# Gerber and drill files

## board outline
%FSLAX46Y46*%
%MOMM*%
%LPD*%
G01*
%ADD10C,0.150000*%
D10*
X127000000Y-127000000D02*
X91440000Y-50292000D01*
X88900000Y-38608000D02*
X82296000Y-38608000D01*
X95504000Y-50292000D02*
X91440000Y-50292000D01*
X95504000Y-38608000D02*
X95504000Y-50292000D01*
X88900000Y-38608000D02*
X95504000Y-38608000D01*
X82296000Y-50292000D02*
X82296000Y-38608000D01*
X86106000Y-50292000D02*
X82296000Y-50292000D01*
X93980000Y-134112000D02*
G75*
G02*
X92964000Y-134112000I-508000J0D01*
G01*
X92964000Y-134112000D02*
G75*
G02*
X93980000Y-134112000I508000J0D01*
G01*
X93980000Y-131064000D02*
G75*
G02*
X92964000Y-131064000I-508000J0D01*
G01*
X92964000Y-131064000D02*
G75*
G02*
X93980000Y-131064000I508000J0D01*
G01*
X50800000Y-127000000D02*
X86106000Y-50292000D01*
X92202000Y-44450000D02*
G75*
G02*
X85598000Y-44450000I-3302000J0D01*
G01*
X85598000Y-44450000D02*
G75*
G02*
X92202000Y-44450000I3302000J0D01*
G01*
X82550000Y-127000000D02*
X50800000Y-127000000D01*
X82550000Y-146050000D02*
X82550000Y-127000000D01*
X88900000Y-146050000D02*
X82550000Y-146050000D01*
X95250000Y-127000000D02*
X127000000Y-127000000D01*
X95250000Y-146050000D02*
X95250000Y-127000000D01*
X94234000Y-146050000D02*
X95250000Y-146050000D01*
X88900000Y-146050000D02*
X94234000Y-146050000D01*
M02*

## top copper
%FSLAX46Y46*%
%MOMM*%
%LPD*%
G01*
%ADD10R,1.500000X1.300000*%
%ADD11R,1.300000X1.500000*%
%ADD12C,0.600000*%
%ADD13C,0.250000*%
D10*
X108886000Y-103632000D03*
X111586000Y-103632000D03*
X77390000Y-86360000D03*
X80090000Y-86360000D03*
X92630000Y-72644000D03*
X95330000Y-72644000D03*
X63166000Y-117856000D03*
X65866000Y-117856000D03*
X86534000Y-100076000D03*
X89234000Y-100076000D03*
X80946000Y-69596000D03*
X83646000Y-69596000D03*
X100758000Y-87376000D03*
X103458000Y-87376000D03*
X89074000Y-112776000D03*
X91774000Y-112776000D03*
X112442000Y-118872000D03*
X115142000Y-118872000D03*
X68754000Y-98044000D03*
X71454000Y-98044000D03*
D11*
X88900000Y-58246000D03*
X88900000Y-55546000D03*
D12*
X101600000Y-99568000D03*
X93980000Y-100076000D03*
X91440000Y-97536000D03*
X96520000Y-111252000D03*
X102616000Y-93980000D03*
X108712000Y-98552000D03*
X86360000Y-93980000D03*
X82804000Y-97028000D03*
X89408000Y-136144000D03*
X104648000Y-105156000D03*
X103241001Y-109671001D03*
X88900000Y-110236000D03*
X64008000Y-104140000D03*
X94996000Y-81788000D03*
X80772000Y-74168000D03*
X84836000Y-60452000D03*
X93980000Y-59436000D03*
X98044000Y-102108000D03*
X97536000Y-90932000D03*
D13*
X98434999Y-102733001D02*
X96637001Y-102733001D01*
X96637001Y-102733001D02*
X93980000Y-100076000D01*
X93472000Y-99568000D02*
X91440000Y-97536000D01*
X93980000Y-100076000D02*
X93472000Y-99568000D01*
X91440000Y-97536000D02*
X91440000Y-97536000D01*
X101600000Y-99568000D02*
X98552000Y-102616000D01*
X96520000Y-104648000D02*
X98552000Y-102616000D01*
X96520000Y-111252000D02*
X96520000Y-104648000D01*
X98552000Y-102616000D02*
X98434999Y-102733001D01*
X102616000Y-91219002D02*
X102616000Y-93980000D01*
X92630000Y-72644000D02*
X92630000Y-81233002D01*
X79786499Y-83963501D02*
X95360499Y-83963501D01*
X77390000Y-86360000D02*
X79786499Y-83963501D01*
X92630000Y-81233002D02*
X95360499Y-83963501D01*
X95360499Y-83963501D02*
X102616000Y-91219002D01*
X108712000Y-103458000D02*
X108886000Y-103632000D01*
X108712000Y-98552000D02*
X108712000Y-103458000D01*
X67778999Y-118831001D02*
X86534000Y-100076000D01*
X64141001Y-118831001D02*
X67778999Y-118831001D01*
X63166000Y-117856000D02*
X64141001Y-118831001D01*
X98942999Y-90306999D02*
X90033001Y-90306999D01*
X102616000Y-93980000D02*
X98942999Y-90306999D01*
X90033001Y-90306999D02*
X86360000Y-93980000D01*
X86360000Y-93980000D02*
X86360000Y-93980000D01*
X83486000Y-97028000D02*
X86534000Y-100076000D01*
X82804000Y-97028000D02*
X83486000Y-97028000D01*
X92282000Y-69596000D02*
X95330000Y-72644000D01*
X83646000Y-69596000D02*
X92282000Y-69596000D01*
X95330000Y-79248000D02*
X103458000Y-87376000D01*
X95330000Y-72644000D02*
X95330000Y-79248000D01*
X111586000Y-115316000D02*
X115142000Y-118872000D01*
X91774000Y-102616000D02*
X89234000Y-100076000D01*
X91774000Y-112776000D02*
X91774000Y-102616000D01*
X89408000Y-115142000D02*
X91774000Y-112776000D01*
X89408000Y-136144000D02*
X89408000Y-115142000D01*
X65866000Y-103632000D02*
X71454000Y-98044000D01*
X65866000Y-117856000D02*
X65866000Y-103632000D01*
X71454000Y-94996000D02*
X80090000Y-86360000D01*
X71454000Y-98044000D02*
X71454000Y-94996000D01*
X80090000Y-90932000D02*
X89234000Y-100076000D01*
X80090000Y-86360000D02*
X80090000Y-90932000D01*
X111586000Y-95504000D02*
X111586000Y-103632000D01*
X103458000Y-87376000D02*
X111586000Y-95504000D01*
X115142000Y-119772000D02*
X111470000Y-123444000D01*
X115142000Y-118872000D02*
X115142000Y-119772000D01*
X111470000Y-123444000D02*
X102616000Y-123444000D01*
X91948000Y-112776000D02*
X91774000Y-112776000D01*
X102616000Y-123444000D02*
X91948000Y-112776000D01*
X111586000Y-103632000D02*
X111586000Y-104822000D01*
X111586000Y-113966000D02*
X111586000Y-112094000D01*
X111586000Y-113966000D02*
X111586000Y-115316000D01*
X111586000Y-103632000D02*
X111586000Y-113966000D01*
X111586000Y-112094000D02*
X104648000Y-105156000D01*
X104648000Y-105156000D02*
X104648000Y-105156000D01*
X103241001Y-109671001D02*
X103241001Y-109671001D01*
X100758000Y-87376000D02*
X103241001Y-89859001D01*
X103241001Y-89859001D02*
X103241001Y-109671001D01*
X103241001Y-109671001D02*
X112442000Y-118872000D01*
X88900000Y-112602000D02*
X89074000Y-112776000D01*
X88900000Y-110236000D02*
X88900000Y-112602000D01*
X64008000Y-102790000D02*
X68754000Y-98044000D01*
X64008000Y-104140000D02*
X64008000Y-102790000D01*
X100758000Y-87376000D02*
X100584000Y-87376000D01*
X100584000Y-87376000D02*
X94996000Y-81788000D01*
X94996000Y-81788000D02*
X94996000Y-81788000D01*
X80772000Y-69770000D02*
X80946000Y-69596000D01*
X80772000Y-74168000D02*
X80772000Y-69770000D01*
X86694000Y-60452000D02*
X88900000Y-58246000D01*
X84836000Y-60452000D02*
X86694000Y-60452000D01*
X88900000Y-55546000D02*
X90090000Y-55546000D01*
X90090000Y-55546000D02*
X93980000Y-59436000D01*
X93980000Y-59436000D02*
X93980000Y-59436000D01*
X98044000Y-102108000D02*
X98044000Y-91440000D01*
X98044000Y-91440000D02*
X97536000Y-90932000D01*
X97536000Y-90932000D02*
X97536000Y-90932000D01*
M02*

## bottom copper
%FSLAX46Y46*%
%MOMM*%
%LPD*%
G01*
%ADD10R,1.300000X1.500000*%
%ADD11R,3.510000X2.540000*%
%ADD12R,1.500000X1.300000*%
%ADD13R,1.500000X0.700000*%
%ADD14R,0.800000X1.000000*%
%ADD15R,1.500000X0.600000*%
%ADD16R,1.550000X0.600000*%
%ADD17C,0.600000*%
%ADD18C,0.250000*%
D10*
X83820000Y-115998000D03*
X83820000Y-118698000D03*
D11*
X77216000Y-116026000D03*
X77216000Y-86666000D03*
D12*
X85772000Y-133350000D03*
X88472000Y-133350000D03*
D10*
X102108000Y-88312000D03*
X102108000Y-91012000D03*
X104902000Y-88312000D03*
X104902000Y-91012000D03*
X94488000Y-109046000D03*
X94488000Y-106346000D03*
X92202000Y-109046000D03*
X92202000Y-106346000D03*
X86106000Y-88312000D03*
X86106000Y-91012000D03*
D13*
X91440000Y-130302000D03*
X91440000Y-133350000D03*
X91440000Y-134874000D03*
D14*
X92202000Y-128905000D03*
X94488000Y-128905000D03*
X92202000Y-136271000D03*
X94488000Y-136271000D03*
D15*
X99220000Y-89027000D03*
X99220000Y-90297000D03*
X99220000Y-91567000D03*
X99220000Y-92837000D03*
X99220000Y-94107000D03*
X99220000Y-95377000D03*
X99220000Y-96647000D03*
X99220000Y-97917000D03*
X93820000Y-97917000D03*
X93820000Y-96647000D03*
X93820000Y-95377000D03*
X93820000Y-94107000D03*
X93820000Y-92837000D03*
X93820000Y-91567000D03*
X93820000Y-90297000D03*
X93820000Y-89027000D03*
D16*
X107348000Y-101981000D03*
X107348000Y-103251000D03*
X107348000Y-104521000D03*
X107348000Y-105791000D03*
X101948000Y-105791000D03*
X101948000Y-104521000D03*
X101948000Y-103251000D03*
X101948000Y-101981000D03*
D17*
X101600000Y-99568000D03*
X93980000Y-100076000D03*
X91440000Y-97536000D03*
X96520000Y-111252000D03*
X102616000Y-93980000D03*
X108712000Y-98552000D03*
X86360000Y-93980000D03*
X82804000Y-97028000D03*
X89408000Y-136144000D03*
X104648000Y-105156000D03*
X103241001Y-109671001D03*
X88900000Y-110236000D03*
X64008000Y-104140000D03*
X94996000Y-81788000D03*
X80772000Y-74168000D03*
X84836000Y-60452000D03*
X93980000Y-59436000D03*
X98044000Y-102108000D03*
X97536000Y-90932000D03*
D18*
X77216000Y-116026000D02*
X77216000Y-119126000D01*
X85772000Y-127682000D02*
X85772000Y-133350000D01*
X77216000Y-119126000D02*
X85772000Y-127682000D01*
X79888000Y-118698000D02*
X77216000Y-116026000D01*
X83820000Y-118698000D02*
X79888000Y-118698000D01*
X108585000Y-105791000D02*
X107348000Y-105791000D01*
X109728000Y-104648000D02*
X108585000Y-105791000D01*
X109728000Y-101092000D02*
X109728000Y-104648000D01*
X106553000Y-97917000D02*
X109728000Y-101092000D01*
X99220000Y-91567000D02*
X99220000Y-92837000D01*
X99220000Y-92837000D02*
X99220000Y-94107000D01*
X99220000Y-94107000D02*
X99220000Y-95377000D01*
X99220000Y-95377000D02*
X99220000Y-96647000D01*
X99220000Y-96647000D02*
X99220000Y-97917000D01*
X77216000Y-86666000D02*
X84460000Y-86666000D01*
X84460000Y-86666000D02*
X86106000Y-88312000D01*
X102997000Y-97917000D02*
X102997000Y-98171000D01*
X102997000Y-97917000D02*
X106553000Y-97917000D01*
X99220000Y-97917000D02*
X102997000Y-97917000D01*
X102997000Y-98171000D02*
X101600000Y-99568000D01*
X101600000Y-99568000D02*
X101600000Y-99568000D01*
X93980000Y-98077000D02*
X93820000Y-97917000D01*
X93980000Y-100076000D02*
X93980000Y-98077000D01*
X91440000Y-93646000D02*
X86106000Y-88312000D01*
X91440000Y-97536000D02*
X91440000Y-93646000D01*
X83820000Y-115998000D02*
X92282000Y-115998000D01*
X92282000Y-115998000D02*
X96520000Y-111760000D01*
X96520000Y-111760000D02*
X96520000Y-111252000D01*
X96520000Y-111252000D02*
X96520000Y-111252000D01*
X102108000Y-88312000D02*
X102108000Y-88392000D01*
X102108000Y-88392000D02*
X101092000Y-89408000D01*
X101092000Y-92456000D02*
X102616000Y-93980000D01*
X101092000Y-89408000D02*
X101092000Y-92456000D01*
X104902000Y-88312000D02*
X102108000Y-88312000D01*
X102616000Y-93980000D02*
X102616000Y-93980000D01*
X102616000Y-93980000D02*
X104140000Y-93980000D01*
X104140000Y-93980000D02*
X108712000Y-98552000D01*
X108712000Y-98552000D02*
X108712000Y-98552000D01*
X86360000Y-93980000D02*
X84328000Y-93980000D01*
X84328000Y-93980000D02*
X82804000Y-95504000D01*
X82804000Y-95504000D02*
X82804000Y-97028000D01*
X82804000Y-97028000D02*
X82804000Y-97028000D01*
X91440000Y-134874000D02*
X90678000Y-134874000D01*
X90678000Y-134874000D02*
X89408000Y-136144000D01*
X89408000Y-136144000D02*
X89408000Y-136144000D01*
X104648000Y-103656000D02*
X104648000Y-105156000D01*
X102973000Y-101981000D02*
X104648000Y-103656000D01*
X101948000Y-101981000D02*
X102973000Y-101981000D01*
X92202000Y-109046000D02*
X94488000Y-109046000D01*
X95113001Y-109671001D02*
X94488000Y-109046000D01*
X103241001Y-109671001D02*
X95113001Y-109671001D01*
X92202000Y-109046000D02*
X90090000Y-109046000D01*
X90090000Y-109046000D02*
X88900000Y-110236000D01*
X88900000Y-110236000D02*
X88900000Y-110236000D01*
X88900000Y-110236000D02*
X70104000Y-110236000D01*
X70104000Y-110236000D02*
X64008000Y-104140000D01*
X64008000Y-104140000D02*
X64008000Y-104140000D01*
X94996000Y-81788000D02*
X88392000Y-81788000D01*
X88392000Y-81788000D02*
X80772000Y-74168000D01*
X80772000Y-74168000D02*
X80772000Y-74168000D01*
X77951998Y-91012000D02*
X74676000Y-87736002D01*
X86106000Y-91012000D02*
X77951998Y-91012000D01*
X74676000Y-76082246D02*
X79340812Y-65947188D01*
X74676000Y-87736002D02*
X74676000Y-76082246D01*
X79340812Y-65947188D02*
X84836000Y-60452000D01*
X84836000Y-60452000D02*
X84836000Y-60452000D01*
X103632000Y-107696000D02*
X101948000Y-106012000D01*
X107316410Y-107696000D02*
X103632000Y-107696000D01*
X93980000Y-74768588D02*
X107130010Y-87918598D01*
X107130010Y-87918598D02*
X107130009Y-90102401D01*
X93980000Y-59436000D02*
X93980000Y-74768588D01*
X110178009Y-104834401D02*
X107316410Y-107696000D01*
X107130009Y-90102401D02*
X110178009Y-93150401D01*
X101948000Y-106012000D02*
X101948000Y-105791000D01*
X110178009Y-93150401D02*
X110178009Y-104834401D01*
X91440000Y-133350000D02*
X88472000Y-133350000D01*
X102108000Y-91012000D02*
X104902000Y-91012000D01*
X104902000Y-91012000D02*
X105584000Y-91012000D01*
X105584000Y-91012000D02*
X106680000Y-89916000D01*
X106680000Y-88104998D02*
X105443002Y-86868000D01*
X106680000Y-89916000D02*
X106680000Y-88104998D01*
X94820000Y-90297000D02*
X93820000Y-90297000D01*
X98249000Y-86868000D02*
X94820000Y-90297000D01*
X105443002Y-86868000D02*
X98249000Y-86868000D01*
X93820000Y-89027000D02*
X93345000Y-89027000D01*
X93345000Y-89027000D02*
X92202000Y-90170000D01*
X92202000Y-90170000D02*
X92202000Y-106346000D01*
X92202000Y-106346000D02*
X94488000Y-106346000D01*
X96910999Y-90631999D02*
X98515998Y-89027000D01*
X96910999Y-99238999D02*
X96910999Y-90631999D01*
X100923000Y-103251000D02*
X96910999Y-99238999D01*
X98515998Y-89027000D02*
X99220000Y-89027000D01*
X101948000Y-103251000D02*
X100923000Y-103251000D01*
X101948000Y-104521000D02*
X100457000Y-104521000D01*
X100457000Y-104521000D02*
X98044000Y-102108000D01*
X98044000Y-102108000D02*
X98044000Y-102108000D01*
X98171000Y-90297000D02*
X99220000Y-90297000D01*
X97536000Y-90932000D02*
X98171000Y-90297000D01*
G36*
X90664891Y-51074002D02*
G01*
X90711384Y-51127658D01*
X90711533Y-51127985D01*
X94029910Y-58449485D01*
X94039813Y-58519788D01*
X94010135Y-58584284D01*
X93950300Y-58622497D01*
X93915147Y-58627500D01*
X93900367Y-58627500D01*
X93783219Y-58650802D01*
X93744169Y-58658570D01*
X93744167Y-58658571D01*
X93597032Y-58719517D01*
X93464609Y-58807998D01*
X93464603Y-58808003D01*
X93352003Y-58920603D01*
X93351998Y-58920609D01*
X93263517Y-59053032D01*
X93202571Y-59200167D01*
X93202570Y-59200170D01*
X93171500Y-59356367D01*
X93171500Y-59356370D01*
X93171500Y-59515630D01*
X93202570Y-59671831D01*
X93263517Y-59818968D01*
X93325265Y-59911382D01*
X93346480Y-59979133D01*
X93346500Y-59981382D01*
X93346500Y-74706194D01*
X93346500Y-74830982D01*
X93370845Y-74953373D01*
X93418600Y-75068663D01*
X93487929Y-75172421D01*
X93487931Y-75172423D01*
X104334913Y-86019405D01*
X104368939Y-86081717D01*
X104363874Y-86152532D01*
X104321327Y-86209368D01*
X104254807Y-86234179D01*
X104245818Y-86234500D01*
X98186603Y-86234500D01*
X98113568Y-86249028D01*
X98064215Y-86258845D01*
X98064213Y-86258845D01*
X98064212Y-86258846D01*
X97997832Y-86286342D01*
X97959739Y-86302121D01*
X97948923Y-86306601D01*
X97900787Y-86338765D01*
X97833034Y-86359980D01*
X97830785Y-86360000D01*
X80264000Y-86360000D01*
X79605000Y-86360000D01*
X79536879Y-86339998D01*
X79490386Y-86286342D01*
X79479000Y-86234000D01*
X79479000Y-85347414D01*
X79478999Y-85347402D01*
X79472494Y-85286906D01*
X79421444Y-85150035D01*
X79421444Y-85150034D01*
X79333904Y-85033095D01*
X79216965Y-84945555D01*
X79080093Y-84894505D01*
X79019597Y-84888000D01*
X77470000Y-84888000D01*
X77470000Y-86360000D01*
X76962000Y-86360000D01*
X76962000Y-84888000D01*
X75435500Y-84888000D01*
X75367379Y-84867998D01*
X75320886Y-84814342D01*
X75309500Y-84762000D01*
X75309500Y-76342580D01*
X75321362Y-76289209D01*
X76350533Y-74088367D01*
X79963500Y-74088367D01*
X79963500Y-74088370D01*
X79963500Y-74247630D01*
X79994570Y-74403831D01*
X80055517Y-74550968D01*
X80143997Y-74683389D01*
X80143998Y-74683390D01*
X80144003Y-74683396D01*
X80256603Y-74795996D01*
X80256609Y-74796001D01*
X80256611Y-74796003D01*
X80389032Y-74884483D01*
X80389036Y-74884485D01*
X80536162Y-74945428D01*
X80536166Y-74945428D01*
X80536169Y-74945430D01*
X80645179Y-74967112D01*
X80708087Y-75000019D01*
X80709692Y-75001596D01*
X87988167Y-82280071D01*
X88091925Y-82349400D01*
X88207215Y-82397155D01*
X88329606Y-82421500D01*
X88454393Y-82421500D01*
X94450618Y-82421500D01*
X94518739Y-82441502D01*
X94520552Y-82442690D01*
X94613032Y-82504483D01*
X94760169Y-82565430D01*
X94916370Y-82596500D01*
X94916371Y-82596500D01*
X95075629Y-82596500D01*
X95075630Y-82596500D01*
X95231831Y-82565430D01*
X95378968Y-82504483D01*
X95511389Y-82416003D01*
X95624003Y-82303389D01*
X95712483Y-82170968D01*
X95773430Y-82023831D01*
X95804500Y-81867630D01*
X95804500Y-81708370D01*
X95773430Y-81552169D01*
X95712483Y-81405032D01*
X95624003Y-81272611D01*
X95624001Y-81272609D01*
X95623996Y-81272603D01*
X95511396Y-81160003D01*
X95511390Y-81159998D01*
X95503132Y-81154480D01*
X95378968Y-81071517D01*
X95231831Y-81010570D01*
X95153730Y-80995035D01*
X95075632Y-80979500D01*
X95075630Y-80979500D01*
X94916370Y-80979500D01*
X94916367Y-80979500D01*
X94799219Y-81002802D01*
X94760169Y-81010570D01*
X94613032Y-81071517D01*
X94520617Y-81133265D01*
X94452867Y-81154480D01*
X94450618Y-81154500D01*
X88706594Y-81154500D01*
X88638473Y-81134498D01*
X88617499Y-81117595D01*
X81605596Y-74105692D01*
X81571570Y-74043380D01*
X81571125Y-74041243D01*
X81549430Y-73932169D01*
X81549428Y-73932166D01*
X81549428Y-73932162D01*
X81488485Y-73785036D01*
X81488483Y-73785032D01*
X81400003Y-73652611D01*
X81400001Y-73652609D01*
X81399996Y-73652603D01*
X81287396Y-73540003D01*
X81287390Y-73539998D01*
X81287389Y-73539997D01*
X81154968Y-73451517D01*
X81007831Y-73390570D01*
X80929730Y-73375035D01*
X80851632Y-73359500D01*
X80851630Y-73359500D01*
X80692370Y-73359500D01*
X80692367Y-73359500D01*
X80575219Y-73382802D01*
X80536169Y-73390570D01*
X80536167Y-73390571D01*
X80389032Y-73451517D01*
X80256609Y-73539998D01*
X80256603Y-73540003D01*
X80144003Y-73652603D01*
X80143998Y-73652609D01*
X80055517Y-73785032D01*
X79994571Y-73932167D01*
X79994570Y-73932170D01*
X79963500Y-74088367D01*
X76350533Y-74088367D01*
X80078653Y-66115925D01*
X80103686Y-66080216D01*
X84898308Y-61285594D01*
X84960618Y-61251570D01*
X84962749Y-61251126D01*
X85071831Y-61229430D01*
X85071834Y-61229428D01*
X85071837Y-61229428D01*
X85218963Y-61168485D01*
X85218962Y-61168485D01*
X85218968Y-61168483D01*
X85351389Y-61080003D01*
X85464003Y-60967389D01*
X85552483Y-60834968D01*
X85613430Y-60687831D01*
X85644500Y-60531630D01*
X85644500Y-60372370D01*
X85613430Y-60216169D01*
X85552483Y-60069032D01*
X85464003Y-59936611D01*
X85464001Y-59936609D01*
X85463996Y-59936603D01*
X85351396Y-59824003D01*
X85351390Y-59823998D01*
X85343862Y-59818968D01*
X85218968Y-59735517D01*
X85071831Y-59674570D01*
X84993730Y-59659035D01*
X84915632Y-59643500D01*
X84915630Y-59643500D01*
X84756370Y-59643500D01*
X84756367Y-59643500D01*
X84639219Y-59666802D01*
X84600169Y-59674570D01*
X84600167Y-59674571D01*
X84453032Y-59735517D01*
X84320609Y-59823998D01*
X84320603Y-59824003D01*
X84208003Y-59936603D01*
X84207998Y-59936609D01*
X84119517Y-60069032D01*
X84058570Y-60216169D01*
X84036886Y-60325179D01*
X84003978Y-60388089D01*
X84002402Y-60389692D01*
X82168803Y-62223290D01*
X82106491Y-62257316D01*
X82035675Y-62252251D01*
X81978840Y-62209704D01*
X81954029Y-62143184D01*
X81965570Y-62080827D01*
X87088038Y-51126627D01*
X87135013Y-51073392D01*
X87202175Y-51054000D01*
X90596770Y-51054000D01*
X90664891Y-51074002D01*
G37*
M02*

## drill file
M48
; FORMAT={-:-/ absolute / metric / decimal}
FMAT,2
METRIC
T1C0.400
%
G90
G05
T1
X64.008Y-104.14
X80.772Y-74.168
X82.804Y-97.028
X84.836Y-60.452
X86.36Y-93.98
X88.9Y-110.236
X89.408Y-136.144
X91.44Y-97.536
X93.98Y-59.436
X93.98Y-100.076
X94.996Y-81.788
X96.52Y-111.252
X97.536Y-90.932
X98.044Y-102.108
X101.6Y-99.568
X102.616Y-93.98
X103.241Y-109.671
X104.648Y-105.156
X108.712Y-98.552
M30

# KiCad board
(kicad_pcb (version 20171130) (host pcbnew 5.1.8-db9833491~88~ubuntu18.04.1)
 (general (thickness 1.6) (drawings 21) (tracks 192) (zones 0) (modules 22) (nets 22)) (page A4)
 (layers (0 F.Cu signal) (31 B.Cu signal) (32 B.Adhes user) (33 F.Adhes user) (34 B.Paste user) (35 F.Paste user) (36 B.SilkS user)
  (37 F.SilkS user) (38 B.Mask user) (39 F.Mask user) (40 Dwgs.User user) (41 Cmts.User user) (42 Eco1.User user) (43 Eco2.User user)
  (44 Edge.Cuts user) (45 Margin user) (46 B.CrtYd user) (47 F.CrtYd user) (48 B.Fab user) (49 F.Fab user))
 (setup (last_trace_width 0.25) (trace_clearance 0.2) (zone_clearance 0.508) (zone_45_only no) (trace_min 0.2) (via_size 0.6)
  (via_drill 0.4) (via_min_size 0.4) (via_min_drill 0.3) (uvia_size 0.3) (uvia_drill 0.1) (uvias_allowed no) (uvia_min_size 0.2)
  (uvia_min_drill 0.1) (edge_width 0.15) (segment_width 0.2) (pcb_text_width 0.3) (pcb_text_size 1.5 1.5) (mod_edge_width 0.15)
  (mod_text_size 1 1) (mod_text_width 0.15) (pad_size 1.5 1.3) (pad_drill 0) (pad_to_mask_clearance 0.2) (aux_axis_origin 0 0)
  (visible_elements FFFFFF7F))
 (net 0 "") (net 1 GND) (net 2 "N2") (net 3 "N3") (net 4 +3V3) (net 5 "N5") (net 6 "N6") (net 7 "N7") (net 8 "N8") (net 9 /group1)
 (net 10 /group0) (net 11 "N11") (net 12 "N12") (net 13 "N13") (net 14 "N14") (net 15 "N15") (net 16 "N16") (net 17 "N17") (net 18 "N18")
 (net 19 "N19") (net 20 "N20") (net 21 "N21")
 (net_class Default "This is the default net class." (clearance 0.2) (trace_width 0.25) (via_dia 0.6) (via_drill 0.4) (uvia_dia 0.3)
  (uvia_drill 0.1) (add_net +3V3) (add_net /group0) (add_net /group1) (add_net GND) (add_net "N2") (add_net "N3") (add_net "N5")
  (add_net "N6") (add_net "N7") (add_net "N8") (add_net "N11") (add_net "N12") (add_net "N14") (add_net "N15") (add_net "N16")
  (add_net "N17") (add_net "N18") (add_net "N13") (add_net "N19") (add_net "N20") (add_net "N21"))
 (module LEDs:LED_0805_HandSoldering (layer B.Cu) (at 83.82 117.348 90)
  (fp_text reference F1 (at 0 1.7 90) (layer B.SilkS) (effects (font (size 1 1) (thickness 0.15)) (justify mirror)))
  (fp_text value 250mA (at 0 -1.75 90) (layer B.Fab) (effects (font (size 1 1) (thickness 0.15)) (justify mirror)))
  (pad 2 smd rect (at 1.35 0 90) (size 1.5 1.3) (layers B.Cu B.Paste B.Mask) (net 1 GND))
  (pad 1 smd rect (at -1.35 0 90) (size 1.5 1.3) (layers B.Cu B.Paste B.Mask) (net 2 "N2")))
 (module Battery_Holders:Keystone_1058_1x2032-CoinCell (layer B.Cu) (at 77.216 101.346 90)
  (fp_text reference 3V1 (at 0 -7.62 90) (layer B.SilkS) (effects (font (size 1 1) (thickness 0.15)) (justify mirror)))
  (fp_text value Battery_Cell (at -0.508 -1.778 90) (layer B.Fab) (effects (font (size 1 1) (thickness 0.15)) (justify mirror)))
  (pad 1 smd rect (at -14.68 0 90) (size 2.54 3.51) (layers B.Cu B.Paste B.Mask) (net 2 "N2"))
  (pad 2 smd rect (at 14.68 0 90) (size 2.54 3.51) (layers B.Cu B.Paste B.Mask) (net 1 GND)))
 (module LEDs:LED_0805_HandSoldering (layer F.Cu) (at 110.236 103.632)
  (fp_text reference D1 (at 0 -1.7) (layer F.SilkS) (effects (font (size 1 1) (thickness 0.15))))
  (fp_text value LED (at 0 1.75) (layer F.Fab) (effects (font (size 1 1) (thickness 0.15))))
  (pad 1 smd rect (at -1.35 0) (size 1.5 1.3) (layers F.Cu F.Paste F.Mask) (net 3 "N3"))
  (pad 2 smd rect (at 1.35 0) (size 1.5 1.3) (layers F.Cu F.Paste F.Mask) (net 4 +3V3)))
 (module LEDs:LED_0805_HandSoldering (layer F.Cu) (at 78.74 86.36)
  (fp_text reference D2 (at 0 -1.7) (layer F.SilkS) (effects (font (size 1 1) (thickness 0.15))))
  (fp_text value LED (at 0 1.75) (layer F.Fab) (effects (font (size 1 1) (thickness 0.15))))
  (pad 1 smd rect (at -1.35 0) (size 1.5 1.3) (layers F.Cu F.Paste F.Mask) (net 3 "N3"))
  (pad 2 smd rect (at 1.35 0) (size 1.5 1.3) (layers F.Cu F.Paste F.Mask) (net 4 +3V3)))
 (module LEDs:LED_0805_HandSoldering (layer F.Cu) (at 93.98 72.644)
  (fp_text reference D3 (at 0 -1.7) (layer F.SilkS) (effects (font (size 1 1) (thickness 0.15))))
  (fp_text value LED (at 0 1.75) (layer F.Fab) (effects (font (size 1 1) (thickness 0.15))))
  (pad 1 smd rect (at -1.35 0) (size 1.5 1.3) (layers F.Cu F.Paste F.Mask) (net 3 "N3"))
  (pad 2 smd rect (at 1.35 0) (size 1.5 1.3) (layers F.Cu F.Paste F.Mask) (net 4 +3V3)))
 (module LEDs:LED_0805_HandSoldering (layer F.Cu) (at 64.516 117.856)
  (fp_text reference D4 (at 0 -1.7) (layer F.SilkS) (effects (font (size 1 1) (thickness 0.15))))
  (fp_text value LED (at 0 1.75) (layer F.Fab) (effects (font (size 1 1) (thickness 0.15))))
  (pad 1 smd rect (at -1.35 0) (size 1.5 1.3) (layers F.Cu F.Paste F.Mask) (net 3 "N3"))
  (pad 2 smd rect (at 1.35 0) (size 1.5 1.3) (layers F.Cu F.Paste F.Mask) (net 4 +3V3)))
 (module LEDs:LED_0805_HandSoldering (layer F.Cu) (at 87.884 100.076)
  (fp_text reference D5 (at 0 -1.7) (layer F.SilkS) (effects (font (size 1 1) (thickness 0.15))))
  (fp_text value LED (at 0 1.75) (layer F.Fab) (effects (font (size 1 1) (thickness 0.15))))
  (pad 1 smd rect (at -1.35 0) (size 1.5 1.3) (layers F.Cu F.Paste F.Mask) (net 3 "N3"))
  (pad 2 smd rect (at 1.35 0) (size 1.5 1.3) (layers F.Cu F.Paste F.Mask) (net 4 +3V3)))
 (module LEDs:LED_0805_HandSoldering (layer F.Cu) (at 82.296 69.596)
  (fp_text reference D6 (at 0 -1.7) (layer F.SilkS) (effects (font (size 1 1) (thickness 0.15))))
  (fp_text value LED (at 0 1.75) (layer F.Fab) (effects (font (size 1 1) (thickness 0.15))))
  (pad 1 smd rect (at -1.35 0) (size 1.5 1.3) (layers F.Cu F.Paste F.Mask) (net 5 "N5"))
  (pad 2 smd rect (at 1.35 0) (size 1.5 1.3) (layers F.Cu F.Paste F.Mask) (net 4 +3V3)))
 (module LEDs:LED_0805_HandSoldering (layer F.Cu) (at 102.108 87.376)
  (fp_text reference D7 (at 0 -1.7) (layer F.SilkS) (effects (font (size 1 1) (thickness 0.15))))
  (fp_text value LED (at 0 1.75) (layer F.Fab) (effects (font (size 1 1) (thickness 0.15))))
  (pad 1 smd rect (at -1.35 0) (size 1.5 1.3) (layers F.Cu F.Paste F.Mask) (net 5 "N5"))
  (pad 2 smd rect (at 1.35 0) (size 1.5 1.3) (layers F.Cu F.Paste F.Mask) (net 4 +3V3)))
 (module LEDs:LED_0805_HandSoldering (layer F.Cu) (at 90.424 112.776)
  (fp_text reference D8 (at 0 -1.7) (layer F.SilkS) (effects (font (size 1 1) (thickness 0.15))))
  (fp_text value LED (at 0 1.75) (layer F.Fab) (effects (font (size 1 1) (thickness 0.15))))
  (pad 1 smd rect (at -1.35 0) (size 1.5 1.3) (layers F.Cu F.Paste F.Mask) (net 5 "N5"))
  (pad 2 smd rect (at 1.35 0) (size 1.5 1.3) (layers F.Cu F.Paste F.Mask) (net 4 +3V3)))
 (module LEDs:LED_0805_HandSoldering (layer F.Cu) (at 113.792 118.872)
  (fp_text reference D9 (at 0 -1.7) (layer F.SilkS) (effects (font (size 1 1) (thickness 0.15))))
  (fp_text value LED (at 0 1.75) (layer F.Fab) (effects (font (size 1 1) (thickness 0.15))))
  (pad 1 smd rect (at -1.35 0) (size 1.5 1.3) (layers F.Cu F.Paste F.Mask) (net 5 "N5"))
  (pad 2 smd rect (at 1.35 0) (size 1.5 1.3) (layers F.Cu F.Paste F.Mask) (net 4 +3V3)))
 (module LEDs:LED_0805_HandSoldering (layer F.Cu) (at 70.104 98.044)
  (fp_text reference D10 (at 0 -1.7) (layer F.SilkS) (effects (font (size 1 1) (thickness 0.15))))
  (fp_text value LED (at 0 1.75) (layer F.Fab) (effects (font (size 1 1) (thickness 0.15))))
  (pad 1 smd rect (at -1.35 0) (size 1.5 1.3) (layers F.Cu F.Paste F.Mask) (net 5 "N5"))
  (pad 2 smd rect (at 1.35 0) (size 1.5 1.3) (layers F.Cu F.Paste F.Mask) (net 4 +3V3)))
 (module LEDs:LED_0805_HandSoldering (layer F.Cu) (at 88.9 56.896 90)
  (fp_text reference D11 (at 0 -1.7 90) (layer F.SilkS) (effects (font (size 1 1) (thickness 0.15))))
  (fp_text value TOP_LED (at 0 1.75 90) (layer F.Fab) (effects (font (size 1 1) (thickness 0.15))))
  (pad 1 smd rect (at -1.35 0 90) (size 1.5 1.3) (layers F.Cu F.Paste F.Mask) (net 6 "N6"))
  (pad 2 smd rect (at 1.35 0 90) (size 1.5 1.3) (layers F.Cu F.Paste F.Mask) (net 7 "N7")))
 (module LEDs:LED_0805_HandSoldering (layer B.Cu) (at 87.122 133.35)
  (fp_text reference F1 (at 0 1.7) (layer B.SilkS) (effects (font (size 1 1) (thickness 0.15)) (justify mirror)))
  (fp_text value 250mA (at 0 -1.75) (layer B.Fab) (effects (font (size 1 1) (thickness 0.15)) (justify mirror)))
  (pad 1 smd rect (at -1.35 0) (size 1.5 1.3) (layers B.Cu B.Paste B.Mask) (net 2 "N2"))
  (pad 2 smd rect (at 1.35 0) (size 1.5 1.3) (layers B.Cu B.Paste B.Mask) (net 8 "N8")))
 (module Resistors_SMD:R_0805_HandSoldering (layer B.Cu) (at 102.108 89.662 270)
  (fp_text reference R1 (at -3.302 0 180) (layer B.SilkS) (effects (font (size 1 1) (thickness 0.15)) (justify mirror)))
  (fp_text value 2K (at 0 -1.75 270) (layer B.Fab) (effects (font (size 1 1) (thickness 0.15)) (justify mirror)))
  (pad 1 smd rect (at -1.35 0 270) (size 1.5 1.3) (layers B.Cu B.Paste B.Mask) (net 3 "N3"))
  (pad 2 smd rect (at 1.35 0 270) (size 1.5 1.3) (layers B.Cu B.Paste B.Mask) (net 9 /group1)))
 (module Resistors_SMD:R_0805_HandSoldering (layer B.Cu) (at 104.902 89.662 270)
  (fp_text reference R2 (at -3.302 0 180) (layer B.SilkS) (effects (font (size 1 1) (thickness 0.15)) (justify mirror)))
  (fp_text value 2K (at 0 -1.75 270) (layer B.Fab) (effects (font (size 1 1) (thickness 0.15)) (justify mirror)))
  (pad 1 smd rect (at -1.35 0 270) (size 1.5 1.3) (layers B.Cu B.Paste B.Mask) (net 3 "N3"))
  (pad 2 smd rect (at 1.35 0 270) (size 1.5 1.3) (layers B.Cu B.Paste B.Mask) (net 9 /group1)))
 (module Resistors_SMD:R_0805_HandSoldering (layer B.Cu) (at 94.488 107.696 90)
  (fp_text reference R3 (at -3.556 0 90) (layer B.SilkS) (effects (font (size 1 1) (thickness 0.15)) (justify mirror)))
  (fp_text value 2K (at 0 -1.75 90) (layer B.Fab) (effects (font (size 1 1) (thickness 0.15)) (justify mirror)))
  (pad 1 smd rect (at -1.35 0 90) (size 1.5 1.3) (layers B.Cu B.Paste B.Mask) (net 5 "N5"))
  (pad 2 smd rect (at 1.35 0 90) (size 1.5 1.3) (layers B.Cu B.Paste B.Mask) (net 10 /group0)))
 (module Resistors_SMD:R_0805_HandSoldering (layer B.Cu) (at 92.202 107.696 90)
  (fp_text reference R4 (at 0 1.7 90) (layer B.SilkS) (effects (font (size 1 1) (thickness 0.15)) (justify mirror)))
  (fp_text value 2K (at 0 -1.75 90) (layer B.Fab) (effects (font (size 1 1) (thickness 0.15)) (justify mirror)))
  (pad 1 smd rect (at -1.35 0 90) (size 1.5 1.3) (layers B.Cu B.Paste B.Mask) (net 5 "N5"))
  (pad 2 smd rect (at 1.35 0 90) (size 1.5 1.3) (layers B.Cu B.Paste B.Mask) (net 10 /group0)))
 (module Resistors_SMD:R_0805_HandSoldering (layer B.Cu) (at 86.106 89.662 270)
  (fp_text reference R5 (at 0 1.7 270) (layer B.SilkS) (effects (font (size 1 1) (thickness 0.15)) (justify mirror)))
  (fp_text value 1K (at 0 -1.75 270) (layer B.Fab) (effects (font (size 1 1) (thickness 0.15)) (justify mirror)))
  (pad 1 smd rect (at -1.35 0 270) (size 1.5 1.3) (layers B.Cu B.Paste B.Mask) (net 1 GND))
  (pad 2 smd rect (at 1.35 0 270) (size 1.5 1.3) (layers B.Cu B.Paste B.Mask) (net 6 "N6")))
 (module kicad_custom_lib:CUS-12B (layer B.Cu) (at 96.266 132.588 270)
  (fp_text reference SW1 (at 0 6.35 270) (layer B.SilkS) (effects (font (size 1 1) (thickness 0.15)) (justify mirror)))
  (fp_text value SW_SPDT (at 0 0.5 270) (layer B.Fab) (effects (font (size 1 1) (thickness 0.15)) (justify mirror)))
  (pad 1 smd rect (at -2.286 4.826 270) (size 0.7 1.5) (layers B.Cu B.Paste B.Mask) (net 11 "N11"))
  (pad 2 smd rect (at 0.762 4.826 270) (size 0.7 1.5) (layers B.Cu B.Paste B.Mask) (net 8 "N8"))
  (pad 3 smd rect (at 2.286 4.826 270) (size 0.7 1.5) (layers B.Cu B.Paste B.Mask) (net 4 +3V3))
  (pad 4 smd rect (at -3.683 4.064 270) (size 1 0.8) (layers B.Cu B.Paste B.Mask))
  (pad 5 smd rect (at -3.683 1.778 270) (size 1 0.8) (layers B.Cu B.Paste B.Mask))
  (pad 6 smd rect (at 3.683 4.064 270) (size 1 0.8) (layers B.Cu B.Paste B.Mask))
  (pad 7 smd rect (at 3.683 1.778 270) (size 1 0.8) (layers B.Cu B.Paste B.Mask)))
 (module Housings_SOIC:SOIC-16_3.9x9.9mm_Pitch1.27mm (layer B.Cu) (at 96.52 93.472 180)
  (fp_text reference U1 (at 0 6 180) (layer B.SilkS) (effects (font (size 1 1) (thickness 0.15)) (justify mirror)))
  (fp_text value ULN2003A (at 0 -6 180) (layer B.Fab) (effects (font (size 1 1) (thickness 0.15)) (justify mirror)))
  (pad 1 smd rect (at -2.7 4.445 180) (size 1.5 0.6) (layers B.Cu B.Paste B.Mask) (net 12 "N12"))
  (pad 2 smd rect (at -2.7 3.175 180) (size 1.5 0.6) (layers B.Cu B.Paste B.Mask) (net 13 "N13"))
  (pad 3 smd rect (at -2.7 1.905 180) (size 1.5 0.6) (layers B.Cu B.Paste B.Mask) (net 1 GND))
  (pad 4 smd rect (at -2.7 0.635 180) (size 1.5 0.6) (layers B.Cu B.Paste B.Mask) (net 1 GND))
  (pad 5 smd rect (at -2.7 -0.635 180) (size 1.5 0.6) (layers B.Cu B.Paste B.Mask) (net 1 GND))
  (pad 6 smd rect (at -2.7 -1.905 180) (size 1.5 0.6) (layers B.Cu B.Paste B.Mask) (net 1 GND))
  (pad 7 smd rect (at -2.7 -3.175 180) (size 1.5 0.6) (layers B.Cu B.Paste B.Mask) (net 1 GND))
  (pad 8 smd rect (at -2.7 -4.445 180) (size 1.5 0.6) (layers B.Cu B.Paste B.Mask) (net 1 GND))
  (pad 9 smd rect (at 2.7 -4.445 180) (size 1.5 0.6) (layers B.Cu B.Paste B.Mask) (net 1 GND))
  (pad 10 smd rect (at 2.7 -3.175 180) (size 1.5 0.6) (layers B.Cu B.Paste B.Mask) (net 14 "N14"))
  (pad 11 smd rect (at 2.7 -1.905 180) (size 1.5 0.6) (layers B.Cu B.Paste B.Mask) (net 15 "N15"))
  (pad 12 smd rect (at 2.7 -0.635 180) (size 1.5 0.6) (layers B.Cu B.Paste B.Mask) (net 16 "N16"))
  (pad 13 smd rect (at 2.7 0.635 180) (size 1.5 0.6) (layers B.Cu B.Paste B.Mask) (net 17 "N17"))
  (pad 14 smd rect (at 2.7 1.905 180) (size 1.5 0.6) (layers B.Cu B.Paste B.Mask) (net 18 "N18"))
  (pad 15 smd rect (at 2.7 3.175 180) (size 1.5 0.6) (layers B.Cu B.Paste B.Mask) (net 9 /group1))
  (pad 16 smd rect (at 2.7 4.445 180) (size 1.5 0.6) (layers B.Cu B.Paste B.Mask) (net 10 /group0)))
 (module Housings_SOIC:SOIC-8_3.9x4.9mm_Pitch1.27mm (layer B.Cu) (at 104.648 103.886 180)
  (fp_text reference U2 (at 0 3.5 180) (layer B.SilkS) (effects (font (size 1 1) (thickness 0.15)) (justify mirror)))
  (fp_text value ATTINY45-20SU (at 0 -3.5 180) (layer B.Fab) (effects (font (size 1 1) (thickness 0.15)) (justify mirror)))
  (pad 1 smd rect (at -2.7 1.905 180) (size 1.55 0.6) (layers B.Cu B.Paste B.Mask) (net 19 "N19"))
  (pad 2 smd rect (at -2.7 0.635 180) (size 1.55 0.6) (layers B.Cu B.Paste B.Mask) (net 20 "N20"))
  (pad 3 smd rect (at -2.7 -0.635 180) (size 1.55 0.6) (layers B.Cu B.Paste B.Mask) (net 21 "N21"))
  (pad 4 smd rect (at -2.7 -1.905 180) (size 1.55 0.6) (layers B.Cu B.Paste B.Mask) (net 1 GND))
  (pad 5 smd rect (at 2.7 -1.905 180) (size 1.55 0.6) (layers B.Cu B.Paste B.Mask) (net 7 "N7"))
  (pad 6 smd rect (at 2.7 -0.635 180) (size 1.55 0.6) (layers B.Cu B.Paste B.Mask) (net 13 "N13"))
  (pad 7 smd rect (at 2.7 0.635 180) (size 1.55 0.6) (layers B.Cu B.Paste B.Mask) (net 12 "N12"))
  (pad 8 smd rect (at 2.7 1.905 180) (size 1.55 0.6) (layers B.Cu B.Paste B.Mask) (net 4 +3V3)))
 (gr_line (start 127 127) (end 91.44 50.292) (layer Edge.Cuts) (width 0.15))
 (gr_line (start 88.9 38.608) (end 82.296 38.608) (layer Edge.Cuts) (width 0.15))
 (gr_line (start 95.504 50.292) (end 91.44 50.292) (layer Edge.Cuts) (width 0.15))
 (gr_line (start 95.504 38.608) (end 95.504 50.292) (layer Edge.Cuts) (width 0.15))
 (gr_line (start 88.9 38.608) (end 95.504 38.608) (layer Edge.Cuts) (width 0.15))
 (gr_line (start 82.296 50.292) (end 82.296 38.608) (layer Edge.Cuts) (width 0.15))
 (gr_line (start 86.106 50.292) (end 82.296 50.292) (layer Edge.Cuts) (width 0.15))
 (gr_circle (center 93.472 134.112) (end 93.472 133.604) (layer Edge.Cuts) (width 0.15))
 (gr_circle (center 93.472 131.064) (end 92.964 131.064) (layer Edge.Cuts) (width 0.15))
 (gr_line (start 50.8 127) (end 86.106 50.292) (angle 90) (layer Edge.Cuts) (width 0.15))
 (gr_circle (center 88.9 44.45) (end 88.9 41.148) (layer Edge.Cuts) (width 0.15))
 (gr_line (start 82.55 127) (end 50.8 127) (angle 90) (layer Edge.Cuts) (width 0.15))
 (gr_line (start 82.55 146.05) (end 82.55 127) (angle 90) (layer Edge.Cuts) (width 0.15))
 (gr_line (start 88.9 146.05) (end 82.55 146.05) (angle 90) (layer Edge.Cuts) (width 0.15))
 (gr_line (start 95.25 127) (end 127 127) (angle 90) (layer Edge.Cuts) (width 0.15))
 (gr_line (start 95.25 146.05) (end 95.25 127) (angle 90) (layer Edge.Cuts) (width 0.15))
 (gr_line (start 94.234 146.05) (end 95.25 146.05) (angle 90) (layer Edge.Cuts) (width 0.15))
 (gr_line (start 88.9 146.05) (end 94.234 146.05) (angle 90) (layer Edge.Cuts) (width 0.15))
 (segment (start 77.216 116.026) (end 77.216 119.126) (width 0.25) (layer B.Cu) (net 2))
 (segment (start 85.772 127.682) (end 85.772 133.35) (width 0.25) (layer B.Cu) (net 2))
 (segment (start 77.216 119.126) (end 85.772 127.682) (width 0.25) (layer B.Cu) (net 2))
 (segment (start 79.888 118.698) (end 77.216 116.026) (width 0.25) (layer B.Cu) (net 2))
 (segment (start 83.82 118.698) (end 79.888 118.698) (width 0.25) (layer B.Cu) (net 2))
 (segment (start 108.585 105.791) (end 107.348 105.791) (width 0.25) (layer B.Cu) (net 1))
 (segment (start 109.728 104.648) (end 108.585 105.791) (width 0.25) (layer B.Cu) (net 1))
 (segment (start 109.728 101.092) (end 109.728 104.648) (width 0.25) (layer B.Cu) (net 1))
 (segment (start 106.553 97.917) (end 109.728 101.092) (width 0.25) (layer B.Cu) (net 1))
 (segment (start 99.22 91.567) (end 99.22 92.837) (width 0.25) (layer B.Cu) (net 1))
 (segment (start 99.22 92.837) (end 99.22 94.107) (width 0.25) (layer B.Cu) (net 1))
 (segment (start 99.22 94.107) (end 99.22 95.377) (width 0.25) (layer B.Cu) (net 1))
 (segment (start 99.22 95.377) (end 99.22 96.647) (width 0.25) (layer B.Cu) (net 1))
 (segment (start 99.22 96.647) (end 99.22 97.917) (width 0.25) (layer B.Cu) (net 1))
 (segment (start 77.216 86.666) (end 84.46 86.666) (width 0.25) (layer B.Cu) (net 1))
 (segment (start 84.46 86.666) (end 86.106 88.312) (width 0.25) (layer B.Cu) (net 1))
 (segment (start 102.997 97.917) (end 102.997 98.171) (width 0.25) (layer B.Cu) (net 1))
 (segment (start 102.997 97.917) (end 106.553 97.917) (width 0.25) (layer B.Cu) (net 1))
 (segment (start 99.22 97.917) (end 102.997 97.917) (width 0.25) (layer B.Cu) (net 1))
 (segment (start 102.997 98.171) (end 101.6 99.568) (width 0.25) (layer B.Cu) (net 1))
 (segment (start 101.6 99.568) (end 101.6 99.568) (width 0.25) (layer B.Cu) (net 1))
 (via (at 101.6 99.568) (size 0.6) (drill 0.4) (layers F.Cu B.Cu) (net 1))
 (segment (start 98.434999 102.733001) (end 96.637001 102.733001) (width 0.25) (layer F.Cu) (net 1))
 (segment (start 96.637001 102.733001) (end 93.98 100.076) (width 0.25) (layer F.Cu) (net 1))
 (segment (start 93.472 99.568) (end 91.44 97.536) (width 0.25) (layer F.Cu) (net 1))
 (segment (start 93.98 100.076) (end 93.472 99.568) (width 0.25) (layer F.Cu) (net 1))
 (via (at 93.98 100.076) (size 0.6) (drill 0.4) (layers F.Cu B.Cu) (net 1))
 (segment (start 91.44 97.536) (end 91.44 97.536) (width 0.25) (layer F.Cu) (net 1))
 (via (at 91.44 97.536) (size 0.6) (drill 0.4) (layers F.Cu B.Cu) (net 1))
 (segment (start 93.98 98.077) (end 93.82 97.917) (width 0.25) (layer B.Cu) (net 1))
 (segment (start 93.98 100.076) (end 93.98 98.077) (width 0.25) (layer B.Cu) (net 1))
 (segment (start 91.44 93.646) (end 86.106 88.312) (width 0.25) (layer B.Cu) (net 1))
 (segment (start 91.44 97.536) (end 91.44 93.646) (width 0.25) (layer B.Cu) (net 1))
 (segment (start 83.82 115.998) (end 92.282 115.998) (width 0.25) (layer B.Cu) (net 1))
 (segment (start 92.282 115.998) (end 96.52 111.76) (width 0.25) (layer B.Cu) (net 1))
 (segment (start 96.52 111.76) (end 96.52 111.252) (width 0.25) (layer B.Cu) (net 1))
 (segment (start 96.52 111.252) (end 96.52 111.252) (width 0.25) (layer B.Cu) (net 1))
 (via (at 96.52 111.252) (size 0.6) (drill 0.4) (layers F.Cu B.Cu) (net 1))
 (segment (start 101.6 99.568) (end 98.552 102.616) (width 0.25) (layer F.Cu) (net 1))
 (segment (start 96.52 104.648) (end 98.552 102.616) (width 0.25) (layer F.Cu) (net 1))
 (segment (start 96.52 111.252) (end 96.52 104.648) (width 0.25) (layer F.Cu) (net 1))
 (segment (start 98.552 102.616) (end 98.434999 102.733001) (width 0.25) (layer F.Cu) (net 1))
 (segment (start 102.108 88.312) (end 102.108 88.392) (width 0.25) (layer B.Cu) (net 3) (status C00000))
 (segment (start 102.108 88.392) (end 101.092 89.408) (width 0.25) (layer B.Cu) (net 3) (status 400000))
 (segment (start 101.092 92.456) (end 102.616 93.98) (width 0.25) (layer B.Cu) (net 3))
 (segment (start 101.092 89.408) (end 101.092 92.456) (width 0.25) (layer B.Cu) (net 3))
 (segment (start 104.902 88.312) (end 102.108 88.312) (width 0.25) (layer B.Cu) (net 3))
 (segment (start 102.616 93.98) (end 102.616 93.98) (width 0.25) (layer B.Cu) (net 3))
 (via (at 102.616 93.98) (size 0.6) (drill 0.4) (layers F.Cu B.Cu) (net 3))
 (segment (start 102.616 91.219002) (end 102.616 93.98) (width 0.25) (layer F.Cu) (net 3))
 (segment (start 92.63 72.644) (end 92.63 81.233002) (width 0.25) (layer F.Cu) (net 3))
 (segment (start 79.786499 83.963501) (end 95.360499 83.963501) (width 0.25) (layer F.Cu) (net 3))
 (segment (start 77.39 86.36) (end 79.786499 83.963501) (width 0.25) (layer F.Cu) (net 3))
 (segment (start 92.63 81.233002) (end 95.360499 83.963501) (width 0.25) (layer F.Cu) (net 3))
 (segment (start 95.360499 83.963501) (end 102.616 91.219002) (width 0.25) (layer F.Cu) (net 3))
 (segment (start 102.616 93.98) (end 104.14 93.98) (width 0.25) (layer B.Cu) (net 3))
 (segment (start 104.14 93.98) (end 108.712 98.552) (width 0.25) (layer B.Cu) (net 3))
 (segment (start 108.712 98.552) (end 108.712 98.552) (width 0.25) (layer B.Cu) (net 3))
 (via (at 108.712 98.552) (size 0.6) (drill 0.4) (layers F.Cu B.Cu) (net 3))
 (segment (start 108.712 103.458) (end 108.886 103.632) (width 0.25) (layer F.Cu) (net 3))
 (segment (start 108.712 98.552) (end 108.712 103.458) (width 0.25) (layer F.Cu) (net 3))
 (segment (start 67.778999 118.831001) (end 86.534 100.076) (width 0.25) (layer F.Cu) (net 3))
 (segment (start 64.141001 118.831001) (end 67.778999 118.831001) (width 0.25) (layer F.Cu) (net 3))
 (segment (start 63.166 117.856) (end 64.141001 118.831001) (width 0.25) (layer F.Cu) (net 3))
 (segment (start 98.942999 90.306999) (end 90.033001 90.306999) (width 0.25) (layer F.Cu) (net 3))
 (segment (start 102.616 93.98) (end 98.942999 90.306999) (width 0.25) (layer F.Cu) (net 3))
 (segment (start 90.033001 90.306999) (end 86.36 93.98) (width 0.25) (layer F.Cu) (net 3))
 (segment (start 86.36 93.98) (end 86.36 93.98) (width 0.25) (layer F.Cu) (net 3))
 (via (at 86.36 93.98) (size 0.6) (drill 0.4) (layers F.Cu B.Cu) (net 3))
 (segment (start 86.36 93.98) (end 84.328 93.98) (width 0.25) (layer B.Cu) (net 3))
 (segment (start 84.328 93.98) (end 82.804 95.504) (width 0.25) (layer B.Cu) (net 3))
 (segment (start 82.804 95.504) (end 82.804 97.028) (width 0.25) (layer B.Cu) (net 3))
 (segment (start 82.804 97.028) (end 82.804 97.028) (width 0.25) (layer B.Cu) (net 3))
 (via (at 82.804 97.028) (size 0.6) (drill 0.4) (layers F.Cu B.Cu) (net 3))
 (segment (start 83.486 97.028) (end 86.534 100.076) (width 0.25) (layer F.Cu) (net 3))
 (segment (start 82.804 97.028) (end 83.486 97.028) (width 0.25) (layer F.Cu) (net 3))
 (segment (start 92.282 69.596) (end 95.33 72.644) (width 0.25) (layer F.Cu) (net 4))
 (segment (start 83.646 69.596) (end 92.282 69.596) (width 0.25) (layer F.Cu) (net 4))
 (segment (start 95.33 79.248) (end 103.458 87.376) (width 0.25) (layer F.Cu) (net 4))
 (segment (start 95.33 72.644) (end 95.33 79.248) (width 0.25) (layer F.Cu) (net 4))
 (segment (start 111.586 115.316) (end 115.142 118.872) (width 0.25) (layer F.Cu) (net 4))
 (segment (start 91.774 102.616) (end 89.234 100.076) (width 0.25) (layer F.Cu) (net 4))
 (segment (start 91.774 112.776) (end 91.774 102.616) (width 0.25) (layer F.Cu) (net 4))
 (segment (start 91.44 134.874) (end 90.678 134.874) (width 0.25) (layer B.Cu) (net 4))
 (segment (start 90.678 134.874) (end 89.408 136.144) (width 0.25) (layer B.Cu) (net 4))
 (segment (start 89.408 136.144) (end 89.408 136.144) (width 0.25) (layer B.Cu) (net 4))
 (via (at 89.408 136.144) (size 0.6) (drill 0.4) (layers F.Cu B.Cu) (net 4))
 (segment (start 89.408 115.142) (end 91.774 112.776) (width 0.25) (layer F.Cu) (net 4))
 (segment (start 89.408 136.144) (end 89.408 115.142) (width 0.25) (layer F.Cu) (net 4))
 (segment (start 65.866 103.632) (end 71.454 98.044) (width 0.25) (layer F.Cu) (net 4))
 (segment (start 65.866 117.856) (end 65.866 103.632) (width 0.25) (layer F.Cu) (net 4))
 (segment (start 71.454 94.996) (end 80.09 86.36) (width 0.25) (layer F.Cu) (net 4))
 (segment (start 71.454 98.044) (end 71.454 94.996) (width 0.25) (layer F.Cu) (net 4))
 (segment (start 80.09 90.932) (end 89.234 100.076) (width 0.25) (layer F.Cu) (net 4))
 (segment (start 80.09 86.36) (end 80.09 90.932) (width 0.25) (layer F.Cu) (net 4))
 (segment (start 111.586 95.504) (end 111.586 103.632) (width 0.25) (layer F.Cu) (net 4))
 (segment (start 103.458 87.376) (end 111.586 95.504) (width 0.25) (layer F.Cu) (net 4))
 (segment (start 115.142 119.772) (end 111.47 123.444) (width 0.25) (layer F.Cu) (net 4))
 (segment (start 115.142 118.872) (end 115.142 119.772) (width 0.25) (layer F.Cu) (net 4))
 (segment (start 111.47 123.444) (end 102.616 123.444) (width 0.25) (layer F.Cu) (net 4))
 (segment (start 91.948 112.776) (end 91.774 112.776) (width 0.25) (layer F.Cu) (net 4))
 (segment (start 102.616 123.444) (end 91.948 112.776) (width 0.25) (layer F.Cu) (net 4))
 (segment (start 111.586 103.632) (end 111.586 104.822) (width 0.25) (layer F.Cu) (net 4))
 (segment (start 111.586 113.966) (end 111.586 112.094) (width 0.25) (layer F.Cu) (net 4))
 (segment (start 111.586 113.966) (end 111.586 115.316) (width 0.25) (layer F.Cu) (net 4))
 (segment (start 111.586 103.632) (end 111.586 113.966) (width 0.25) (layer F.Cu) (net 4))
 (segment (start 111.586 112.094) (end 104.648 105.156) (width 0.25) (layer F.Cu) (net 4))
 (segment (start 104.648 105.156) (end 104.648 105.156) (width 0.25) (layer F.Cu) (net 4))
 (via (at 104.648 105.156) (size 0.6) (drill 0.4) (layers F.Cu B.Cu) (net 4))
 (segment (start 104.648 103.656) (end 104.648 105.156) (width 0.25) (layer B.Cu) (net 4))
 (segment (start 102.973 101.981) (end 104.648 103.656) (width 0.25) (layer B.Cu) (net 4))
 (segment (start 101.948 101.981) (end 102.973 101.981) (width 0.25) (layer B.Cu) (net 4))
 (segment (start 92.202 109.046) (end 94.488 109.046) (width 0.25) (layer B.Cu) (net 5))
 (segment (start 103.241001 109.671001) (end 103.241001 109.671001) (width 0.25) (layer F.Cu) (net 5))
 (segment (start 100.758 87.376) (end 103.241001 89.859001) (width 0.25) (layer F.Cu) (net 5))
 (segment (start 103.241001 89.859001) (end 103.241001 109.671001) (width 0.25) (layer F.Cu) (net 5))
 (segment (start 103.241001 109.671001) (end 112.442 118.872) (width 0.25) (layer F.Cu) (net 5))
 (via (at 103.241001 109.671001) (size 0.6) (drill 0.4) (layers F.Cu B.Cu) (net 5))
 (segment (start 95.113001 109.671001) (end 94.488 109.046) (width 0.25) (layer B.Cu) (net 5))
 (segment (start 103.241001 109.671001) (end 95.113001 109.671001) (width 0.25) (layer B.Cu) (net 5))
 (segment (start 92.202 109.046) (end 90.09 109.046) (width 0.25) (layer B.Cu) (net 5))
 (segment (start 90.09 109.046) (end 88.9 110.236) (width 0.25) (layer B.Cu) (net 5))
 (segment (start 88.9 110.236) (end 88.9 110.236) (width 0.25) (layer B.Cu) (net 5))
 (via (at 88.9 110.236) (size 0.6) (drill 0.4) (layers F.Cu B.Cu) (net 5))
 (segment (start 88.9 112.602) (end 89.074 112.776) (width 0.25) (layer F.Cu) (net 5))
 (segment (start 88.9 110.236) (end 88.9 112.602) (width 0.25) (layer F.Cu) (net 5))
 (segment (start 88.9 110.236) (end 70.104 110.236) (width 0.25) (layer B.Cu) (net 5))
 (segment (start 70.104 110.236) (end 64.008 104.14) (width 0.25) (layer B.Cu) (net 5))
 (segment (start 64.008 104.14) (end 64.008 104.14) (width 0.25) (layer B.Cu) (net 5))
 (via (at 64.008 104.14) (size 0.6) (drill 0.4) (layers F.Cu B.Cu) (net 5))
 (segment (start 64.008 102.79) (end 68.754 98.044) (width 0.25) (layer F.Cu) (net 5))
 (segment (start 64.008 104.14) (end 64.008 102.79) (width 0.25) (layer F.Cu) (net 5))
 (segment (start 100.758 87.376) (end 100.584 87.376) (width 0.25) (layer F.Cu) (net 5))
 (segment (start 100.584 87.376) (end 94.996 81.788) (width 0.25) (layer F.Cu) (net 5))
 (segment (start 94.996 81.788) (end 94.996 81.788) (width 0.25) (layer F.Cu) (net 5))
 (via (at 94.996 81.788) (size 0.6) (drill 0.4) (layers F.Cu B.Cu) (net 5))
 (segment (start 94.996 81.788) (end 88.392 81.788) (width 0.25) (layer B.Cu) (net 5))
 (segment (start 88.392 81.788) (end 80.772 74.168) (width 0.25) (layer B.Cu) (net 5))
 (segment (start 80.772 74.168) (end 80.772 74.168) (width 0.25) (layer B.Cu) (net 5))
 (via (at 80.772 74.168) (size 0.6) (drill 0.4) (layers F.Cu B.Cu) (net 5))
 (segment (start 80.772 69.77) (end 80.946 69.596) (width 0.25) (layer F.Cu) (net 5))
 (segment (start 80.772 74.168) (end 80.772 69.77) (width 0.25) (layer F.Cu) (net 5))
 (segment (start 77.951998 91.012) (end 74.676 87.736002) (width 0.25) (layer B.Cu) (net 6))
 (segment (start 86.106 91.012) (end 77.951998 91.012) (width 0.25) (layer B.Cu) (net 6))
 (segment (start 74.676 76.082246) (end 79.340812 65.947188) (width 0.25) (layer B.Cu) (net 6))
 (segment (start 74.676 87.736002) (end 74.676 76.082246) (width 0.25) (layer B.Cu) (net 6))
 (segment (start 79.340812 65.947188) (end 84.836 60.452) (width 0.25) (layer B.Cu) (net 6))
 (segment (start 84.836 60.452) (end 84.836 60.452) (width 0.25) (layer B.Cu) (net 6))
 (via (at 84.836 60.452) (size 0.6) (drill 0.4) (layers F.Cu B.Cu) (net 6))
 (segment (start 86.694 60.452) (end 88.9 58.246) (width 0.25) (layer F.Cu) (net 6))
 (segment (start 84.836 60.452) (end 86.694 60.452) (width 0.25) (layer F.Cu) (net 6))
 (segment (start 88.9 55.546) (end 90.09 55.546) (width 0.25) (layer F.Cu) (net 7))
 (segment (start 90.09 55.546) (end 93.98 59.436) (width 0.25) (layer F.Cu) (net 7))
 (segment (start 93.98 59.436) (end 93.98 59.436) (width 0.25) (layer F.Cu) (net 7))
 (via (at 93.98 59.436) (size 0.6) (drill 0.4) (layers F.Cu B.Cu) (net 7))
 (segment (start 103.632 107.696) (end 101.948 106.012) (width 0.25) (layer B.Cu) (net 7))
 (segment (start 107.31641 107.696) (end 103.632 107.696) (width 0.25) (layer B.Cu) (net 7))
 (segment (start 93.98 74.768588) (end 107.13001 87.918598) (width 0.25) (layer B.Cu) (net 7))
 (segment (start 107.13001 87.918598) (end 107.130009 90.102401) (width 0.25) (layer B.Cu) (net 7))
 (segment (start 93.98 59.436) (end 93.98 74.768588) (width 0.25) (layer B.Cu) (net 7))
 (segment (start 110.178009 104.834401) (end 107.31641 107.696) (width 0.25) (layer B.Cu) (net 7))
 (segment (start 107.130009 90.102401) (end 110.178009 93.150401) (width 0.25) (layer B.Cu) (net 7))
 (segment (start 101.948 106.012) (end 101.948 105.791) (width 0.25) (layer B.Cu) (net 7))
 (segment (start 110.178009 93.150401) (end 110.178009 104.834401) (width 0.25) (layer B.Cu) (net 7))
 (segment (start 91.44 133.35) (end 88.472 133.35) (width 0.25) (layer B.Cu) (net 8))
 (segment (start 102.108 91.012) (end 104.902 91.012) (width 0.25) (layer B.Cu) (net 9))
 (segment (start 104.902 91.012) (end 105.584 91.012) (width 0.25) (layer B.Cu) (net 9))
 (segment (start 105.584 91.012) (end 106.68 89.916) (width 0.25) (layer B.Cu) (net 9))
 (segment (start 106.68 88.104998) (end 105.443002 86.868) (width 0.25) (layer B.Cu) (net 9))
 (segment (start 106.68 89.916) (end 106.68 88.104998) (width 0.25) (layer B.Cu) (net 9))
 (segment (start 94.82 90.297) (end 93.82 90.297) (width 0.25) (layer B.Cu) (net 9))
 (segment (start 98.249 86.868) (end 94.82 90.297) (width 0.25) (layer B.Cu) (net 9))
 (segment (start 105.443002 86.868) (end 98.249 86.868) (width 0.25) (layer B.Cu) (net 9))
 (segment (start 93.82 89.027) (end 93.345 89.027) (width 0.25) (layer B.Cu) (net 10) (status C00000))
 (segment (start 93.345 89.027) (end 92.202 90.17) (width 0.25) (layer B.Cu) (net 10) (status 400000))
 (segment (start 92.202 90.17) (end 92.202 106.346) (width 0.25) (layer B.Cu) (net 10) (status 800000))
 (segment (start 92.202 106.346) (end 94.488 106.346) (width 0.25) (layer B.Cu) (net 10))
 (segment (start 96.910999 90.631999) (end 98.515998 89.027) (width 0.25) (layer B.Cu) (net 12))
 (segment (start 96.910999 99.238999) (end 96.910999 90.631999) (width 0.25) (layer B.Cu) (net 12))
 (segment (start 100.923 103.251) (end 96.910999 99.238999) (width 0.25) (layer B.Cu) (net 12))
 (segment (start 98.515998 89.027) (end 99.22 89.027) (width 0.25) (layer B.Cu) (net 12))
 (segment (start 101.948 103.251) (end 100.923 103.251) (width 0.25) (layer B.Cu) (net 12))
 (segment (start 101.948 104.521) (end 100.457 104.521) (width 0.25) (layer B.Cu) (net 13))
 (segment (start 100.457 104.521) (end 98.044 102.108) (width 0.25) (layer B.Cu) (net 13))
 (segment (start 98.044 102.108) (end 98.044 102.108) (width 0.25) (layer B.Cu) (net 13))
 (via (at 98.044 102.108) (size 0.6) (drill 0.4) (layers F.Cu B.Cu) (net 13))
 (segment (start 98.044 102.108) (end 98.044 91.44) (width 0.25) (layer F.Cu) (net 13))
 (segment (start 98.044 91.44) (end 97.536 90.932) (width 0.25) (layer F.Cu) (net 13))
 (segment (start 97.536 90.932) (end 97.536 90.932) (width 0.25) (layer F.Cu) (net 13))
 (via (at 97.536 90.932) (size 0.6) (drill 0.4) (layers F.Cu B.Cu) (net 13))
 (segment (start 98.171 90.297) (end 99.22 90.297) (width 0.25) (layer B.Cu) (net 13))
 (segment (start 97.536 90.932) (end 98.171 90.297) (width 0.25) (layer B.Cu) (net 13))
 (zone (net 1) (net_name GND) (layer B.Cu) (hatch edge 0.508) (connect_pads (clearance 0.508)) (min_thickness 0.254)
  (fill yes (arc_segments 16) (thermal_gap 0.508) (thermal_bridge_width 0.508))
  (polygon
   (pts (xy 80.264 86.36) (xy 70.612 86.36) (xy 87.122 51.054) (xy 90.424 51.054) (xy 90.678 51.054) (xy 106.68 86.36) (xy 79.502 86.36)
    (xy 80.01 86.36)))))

